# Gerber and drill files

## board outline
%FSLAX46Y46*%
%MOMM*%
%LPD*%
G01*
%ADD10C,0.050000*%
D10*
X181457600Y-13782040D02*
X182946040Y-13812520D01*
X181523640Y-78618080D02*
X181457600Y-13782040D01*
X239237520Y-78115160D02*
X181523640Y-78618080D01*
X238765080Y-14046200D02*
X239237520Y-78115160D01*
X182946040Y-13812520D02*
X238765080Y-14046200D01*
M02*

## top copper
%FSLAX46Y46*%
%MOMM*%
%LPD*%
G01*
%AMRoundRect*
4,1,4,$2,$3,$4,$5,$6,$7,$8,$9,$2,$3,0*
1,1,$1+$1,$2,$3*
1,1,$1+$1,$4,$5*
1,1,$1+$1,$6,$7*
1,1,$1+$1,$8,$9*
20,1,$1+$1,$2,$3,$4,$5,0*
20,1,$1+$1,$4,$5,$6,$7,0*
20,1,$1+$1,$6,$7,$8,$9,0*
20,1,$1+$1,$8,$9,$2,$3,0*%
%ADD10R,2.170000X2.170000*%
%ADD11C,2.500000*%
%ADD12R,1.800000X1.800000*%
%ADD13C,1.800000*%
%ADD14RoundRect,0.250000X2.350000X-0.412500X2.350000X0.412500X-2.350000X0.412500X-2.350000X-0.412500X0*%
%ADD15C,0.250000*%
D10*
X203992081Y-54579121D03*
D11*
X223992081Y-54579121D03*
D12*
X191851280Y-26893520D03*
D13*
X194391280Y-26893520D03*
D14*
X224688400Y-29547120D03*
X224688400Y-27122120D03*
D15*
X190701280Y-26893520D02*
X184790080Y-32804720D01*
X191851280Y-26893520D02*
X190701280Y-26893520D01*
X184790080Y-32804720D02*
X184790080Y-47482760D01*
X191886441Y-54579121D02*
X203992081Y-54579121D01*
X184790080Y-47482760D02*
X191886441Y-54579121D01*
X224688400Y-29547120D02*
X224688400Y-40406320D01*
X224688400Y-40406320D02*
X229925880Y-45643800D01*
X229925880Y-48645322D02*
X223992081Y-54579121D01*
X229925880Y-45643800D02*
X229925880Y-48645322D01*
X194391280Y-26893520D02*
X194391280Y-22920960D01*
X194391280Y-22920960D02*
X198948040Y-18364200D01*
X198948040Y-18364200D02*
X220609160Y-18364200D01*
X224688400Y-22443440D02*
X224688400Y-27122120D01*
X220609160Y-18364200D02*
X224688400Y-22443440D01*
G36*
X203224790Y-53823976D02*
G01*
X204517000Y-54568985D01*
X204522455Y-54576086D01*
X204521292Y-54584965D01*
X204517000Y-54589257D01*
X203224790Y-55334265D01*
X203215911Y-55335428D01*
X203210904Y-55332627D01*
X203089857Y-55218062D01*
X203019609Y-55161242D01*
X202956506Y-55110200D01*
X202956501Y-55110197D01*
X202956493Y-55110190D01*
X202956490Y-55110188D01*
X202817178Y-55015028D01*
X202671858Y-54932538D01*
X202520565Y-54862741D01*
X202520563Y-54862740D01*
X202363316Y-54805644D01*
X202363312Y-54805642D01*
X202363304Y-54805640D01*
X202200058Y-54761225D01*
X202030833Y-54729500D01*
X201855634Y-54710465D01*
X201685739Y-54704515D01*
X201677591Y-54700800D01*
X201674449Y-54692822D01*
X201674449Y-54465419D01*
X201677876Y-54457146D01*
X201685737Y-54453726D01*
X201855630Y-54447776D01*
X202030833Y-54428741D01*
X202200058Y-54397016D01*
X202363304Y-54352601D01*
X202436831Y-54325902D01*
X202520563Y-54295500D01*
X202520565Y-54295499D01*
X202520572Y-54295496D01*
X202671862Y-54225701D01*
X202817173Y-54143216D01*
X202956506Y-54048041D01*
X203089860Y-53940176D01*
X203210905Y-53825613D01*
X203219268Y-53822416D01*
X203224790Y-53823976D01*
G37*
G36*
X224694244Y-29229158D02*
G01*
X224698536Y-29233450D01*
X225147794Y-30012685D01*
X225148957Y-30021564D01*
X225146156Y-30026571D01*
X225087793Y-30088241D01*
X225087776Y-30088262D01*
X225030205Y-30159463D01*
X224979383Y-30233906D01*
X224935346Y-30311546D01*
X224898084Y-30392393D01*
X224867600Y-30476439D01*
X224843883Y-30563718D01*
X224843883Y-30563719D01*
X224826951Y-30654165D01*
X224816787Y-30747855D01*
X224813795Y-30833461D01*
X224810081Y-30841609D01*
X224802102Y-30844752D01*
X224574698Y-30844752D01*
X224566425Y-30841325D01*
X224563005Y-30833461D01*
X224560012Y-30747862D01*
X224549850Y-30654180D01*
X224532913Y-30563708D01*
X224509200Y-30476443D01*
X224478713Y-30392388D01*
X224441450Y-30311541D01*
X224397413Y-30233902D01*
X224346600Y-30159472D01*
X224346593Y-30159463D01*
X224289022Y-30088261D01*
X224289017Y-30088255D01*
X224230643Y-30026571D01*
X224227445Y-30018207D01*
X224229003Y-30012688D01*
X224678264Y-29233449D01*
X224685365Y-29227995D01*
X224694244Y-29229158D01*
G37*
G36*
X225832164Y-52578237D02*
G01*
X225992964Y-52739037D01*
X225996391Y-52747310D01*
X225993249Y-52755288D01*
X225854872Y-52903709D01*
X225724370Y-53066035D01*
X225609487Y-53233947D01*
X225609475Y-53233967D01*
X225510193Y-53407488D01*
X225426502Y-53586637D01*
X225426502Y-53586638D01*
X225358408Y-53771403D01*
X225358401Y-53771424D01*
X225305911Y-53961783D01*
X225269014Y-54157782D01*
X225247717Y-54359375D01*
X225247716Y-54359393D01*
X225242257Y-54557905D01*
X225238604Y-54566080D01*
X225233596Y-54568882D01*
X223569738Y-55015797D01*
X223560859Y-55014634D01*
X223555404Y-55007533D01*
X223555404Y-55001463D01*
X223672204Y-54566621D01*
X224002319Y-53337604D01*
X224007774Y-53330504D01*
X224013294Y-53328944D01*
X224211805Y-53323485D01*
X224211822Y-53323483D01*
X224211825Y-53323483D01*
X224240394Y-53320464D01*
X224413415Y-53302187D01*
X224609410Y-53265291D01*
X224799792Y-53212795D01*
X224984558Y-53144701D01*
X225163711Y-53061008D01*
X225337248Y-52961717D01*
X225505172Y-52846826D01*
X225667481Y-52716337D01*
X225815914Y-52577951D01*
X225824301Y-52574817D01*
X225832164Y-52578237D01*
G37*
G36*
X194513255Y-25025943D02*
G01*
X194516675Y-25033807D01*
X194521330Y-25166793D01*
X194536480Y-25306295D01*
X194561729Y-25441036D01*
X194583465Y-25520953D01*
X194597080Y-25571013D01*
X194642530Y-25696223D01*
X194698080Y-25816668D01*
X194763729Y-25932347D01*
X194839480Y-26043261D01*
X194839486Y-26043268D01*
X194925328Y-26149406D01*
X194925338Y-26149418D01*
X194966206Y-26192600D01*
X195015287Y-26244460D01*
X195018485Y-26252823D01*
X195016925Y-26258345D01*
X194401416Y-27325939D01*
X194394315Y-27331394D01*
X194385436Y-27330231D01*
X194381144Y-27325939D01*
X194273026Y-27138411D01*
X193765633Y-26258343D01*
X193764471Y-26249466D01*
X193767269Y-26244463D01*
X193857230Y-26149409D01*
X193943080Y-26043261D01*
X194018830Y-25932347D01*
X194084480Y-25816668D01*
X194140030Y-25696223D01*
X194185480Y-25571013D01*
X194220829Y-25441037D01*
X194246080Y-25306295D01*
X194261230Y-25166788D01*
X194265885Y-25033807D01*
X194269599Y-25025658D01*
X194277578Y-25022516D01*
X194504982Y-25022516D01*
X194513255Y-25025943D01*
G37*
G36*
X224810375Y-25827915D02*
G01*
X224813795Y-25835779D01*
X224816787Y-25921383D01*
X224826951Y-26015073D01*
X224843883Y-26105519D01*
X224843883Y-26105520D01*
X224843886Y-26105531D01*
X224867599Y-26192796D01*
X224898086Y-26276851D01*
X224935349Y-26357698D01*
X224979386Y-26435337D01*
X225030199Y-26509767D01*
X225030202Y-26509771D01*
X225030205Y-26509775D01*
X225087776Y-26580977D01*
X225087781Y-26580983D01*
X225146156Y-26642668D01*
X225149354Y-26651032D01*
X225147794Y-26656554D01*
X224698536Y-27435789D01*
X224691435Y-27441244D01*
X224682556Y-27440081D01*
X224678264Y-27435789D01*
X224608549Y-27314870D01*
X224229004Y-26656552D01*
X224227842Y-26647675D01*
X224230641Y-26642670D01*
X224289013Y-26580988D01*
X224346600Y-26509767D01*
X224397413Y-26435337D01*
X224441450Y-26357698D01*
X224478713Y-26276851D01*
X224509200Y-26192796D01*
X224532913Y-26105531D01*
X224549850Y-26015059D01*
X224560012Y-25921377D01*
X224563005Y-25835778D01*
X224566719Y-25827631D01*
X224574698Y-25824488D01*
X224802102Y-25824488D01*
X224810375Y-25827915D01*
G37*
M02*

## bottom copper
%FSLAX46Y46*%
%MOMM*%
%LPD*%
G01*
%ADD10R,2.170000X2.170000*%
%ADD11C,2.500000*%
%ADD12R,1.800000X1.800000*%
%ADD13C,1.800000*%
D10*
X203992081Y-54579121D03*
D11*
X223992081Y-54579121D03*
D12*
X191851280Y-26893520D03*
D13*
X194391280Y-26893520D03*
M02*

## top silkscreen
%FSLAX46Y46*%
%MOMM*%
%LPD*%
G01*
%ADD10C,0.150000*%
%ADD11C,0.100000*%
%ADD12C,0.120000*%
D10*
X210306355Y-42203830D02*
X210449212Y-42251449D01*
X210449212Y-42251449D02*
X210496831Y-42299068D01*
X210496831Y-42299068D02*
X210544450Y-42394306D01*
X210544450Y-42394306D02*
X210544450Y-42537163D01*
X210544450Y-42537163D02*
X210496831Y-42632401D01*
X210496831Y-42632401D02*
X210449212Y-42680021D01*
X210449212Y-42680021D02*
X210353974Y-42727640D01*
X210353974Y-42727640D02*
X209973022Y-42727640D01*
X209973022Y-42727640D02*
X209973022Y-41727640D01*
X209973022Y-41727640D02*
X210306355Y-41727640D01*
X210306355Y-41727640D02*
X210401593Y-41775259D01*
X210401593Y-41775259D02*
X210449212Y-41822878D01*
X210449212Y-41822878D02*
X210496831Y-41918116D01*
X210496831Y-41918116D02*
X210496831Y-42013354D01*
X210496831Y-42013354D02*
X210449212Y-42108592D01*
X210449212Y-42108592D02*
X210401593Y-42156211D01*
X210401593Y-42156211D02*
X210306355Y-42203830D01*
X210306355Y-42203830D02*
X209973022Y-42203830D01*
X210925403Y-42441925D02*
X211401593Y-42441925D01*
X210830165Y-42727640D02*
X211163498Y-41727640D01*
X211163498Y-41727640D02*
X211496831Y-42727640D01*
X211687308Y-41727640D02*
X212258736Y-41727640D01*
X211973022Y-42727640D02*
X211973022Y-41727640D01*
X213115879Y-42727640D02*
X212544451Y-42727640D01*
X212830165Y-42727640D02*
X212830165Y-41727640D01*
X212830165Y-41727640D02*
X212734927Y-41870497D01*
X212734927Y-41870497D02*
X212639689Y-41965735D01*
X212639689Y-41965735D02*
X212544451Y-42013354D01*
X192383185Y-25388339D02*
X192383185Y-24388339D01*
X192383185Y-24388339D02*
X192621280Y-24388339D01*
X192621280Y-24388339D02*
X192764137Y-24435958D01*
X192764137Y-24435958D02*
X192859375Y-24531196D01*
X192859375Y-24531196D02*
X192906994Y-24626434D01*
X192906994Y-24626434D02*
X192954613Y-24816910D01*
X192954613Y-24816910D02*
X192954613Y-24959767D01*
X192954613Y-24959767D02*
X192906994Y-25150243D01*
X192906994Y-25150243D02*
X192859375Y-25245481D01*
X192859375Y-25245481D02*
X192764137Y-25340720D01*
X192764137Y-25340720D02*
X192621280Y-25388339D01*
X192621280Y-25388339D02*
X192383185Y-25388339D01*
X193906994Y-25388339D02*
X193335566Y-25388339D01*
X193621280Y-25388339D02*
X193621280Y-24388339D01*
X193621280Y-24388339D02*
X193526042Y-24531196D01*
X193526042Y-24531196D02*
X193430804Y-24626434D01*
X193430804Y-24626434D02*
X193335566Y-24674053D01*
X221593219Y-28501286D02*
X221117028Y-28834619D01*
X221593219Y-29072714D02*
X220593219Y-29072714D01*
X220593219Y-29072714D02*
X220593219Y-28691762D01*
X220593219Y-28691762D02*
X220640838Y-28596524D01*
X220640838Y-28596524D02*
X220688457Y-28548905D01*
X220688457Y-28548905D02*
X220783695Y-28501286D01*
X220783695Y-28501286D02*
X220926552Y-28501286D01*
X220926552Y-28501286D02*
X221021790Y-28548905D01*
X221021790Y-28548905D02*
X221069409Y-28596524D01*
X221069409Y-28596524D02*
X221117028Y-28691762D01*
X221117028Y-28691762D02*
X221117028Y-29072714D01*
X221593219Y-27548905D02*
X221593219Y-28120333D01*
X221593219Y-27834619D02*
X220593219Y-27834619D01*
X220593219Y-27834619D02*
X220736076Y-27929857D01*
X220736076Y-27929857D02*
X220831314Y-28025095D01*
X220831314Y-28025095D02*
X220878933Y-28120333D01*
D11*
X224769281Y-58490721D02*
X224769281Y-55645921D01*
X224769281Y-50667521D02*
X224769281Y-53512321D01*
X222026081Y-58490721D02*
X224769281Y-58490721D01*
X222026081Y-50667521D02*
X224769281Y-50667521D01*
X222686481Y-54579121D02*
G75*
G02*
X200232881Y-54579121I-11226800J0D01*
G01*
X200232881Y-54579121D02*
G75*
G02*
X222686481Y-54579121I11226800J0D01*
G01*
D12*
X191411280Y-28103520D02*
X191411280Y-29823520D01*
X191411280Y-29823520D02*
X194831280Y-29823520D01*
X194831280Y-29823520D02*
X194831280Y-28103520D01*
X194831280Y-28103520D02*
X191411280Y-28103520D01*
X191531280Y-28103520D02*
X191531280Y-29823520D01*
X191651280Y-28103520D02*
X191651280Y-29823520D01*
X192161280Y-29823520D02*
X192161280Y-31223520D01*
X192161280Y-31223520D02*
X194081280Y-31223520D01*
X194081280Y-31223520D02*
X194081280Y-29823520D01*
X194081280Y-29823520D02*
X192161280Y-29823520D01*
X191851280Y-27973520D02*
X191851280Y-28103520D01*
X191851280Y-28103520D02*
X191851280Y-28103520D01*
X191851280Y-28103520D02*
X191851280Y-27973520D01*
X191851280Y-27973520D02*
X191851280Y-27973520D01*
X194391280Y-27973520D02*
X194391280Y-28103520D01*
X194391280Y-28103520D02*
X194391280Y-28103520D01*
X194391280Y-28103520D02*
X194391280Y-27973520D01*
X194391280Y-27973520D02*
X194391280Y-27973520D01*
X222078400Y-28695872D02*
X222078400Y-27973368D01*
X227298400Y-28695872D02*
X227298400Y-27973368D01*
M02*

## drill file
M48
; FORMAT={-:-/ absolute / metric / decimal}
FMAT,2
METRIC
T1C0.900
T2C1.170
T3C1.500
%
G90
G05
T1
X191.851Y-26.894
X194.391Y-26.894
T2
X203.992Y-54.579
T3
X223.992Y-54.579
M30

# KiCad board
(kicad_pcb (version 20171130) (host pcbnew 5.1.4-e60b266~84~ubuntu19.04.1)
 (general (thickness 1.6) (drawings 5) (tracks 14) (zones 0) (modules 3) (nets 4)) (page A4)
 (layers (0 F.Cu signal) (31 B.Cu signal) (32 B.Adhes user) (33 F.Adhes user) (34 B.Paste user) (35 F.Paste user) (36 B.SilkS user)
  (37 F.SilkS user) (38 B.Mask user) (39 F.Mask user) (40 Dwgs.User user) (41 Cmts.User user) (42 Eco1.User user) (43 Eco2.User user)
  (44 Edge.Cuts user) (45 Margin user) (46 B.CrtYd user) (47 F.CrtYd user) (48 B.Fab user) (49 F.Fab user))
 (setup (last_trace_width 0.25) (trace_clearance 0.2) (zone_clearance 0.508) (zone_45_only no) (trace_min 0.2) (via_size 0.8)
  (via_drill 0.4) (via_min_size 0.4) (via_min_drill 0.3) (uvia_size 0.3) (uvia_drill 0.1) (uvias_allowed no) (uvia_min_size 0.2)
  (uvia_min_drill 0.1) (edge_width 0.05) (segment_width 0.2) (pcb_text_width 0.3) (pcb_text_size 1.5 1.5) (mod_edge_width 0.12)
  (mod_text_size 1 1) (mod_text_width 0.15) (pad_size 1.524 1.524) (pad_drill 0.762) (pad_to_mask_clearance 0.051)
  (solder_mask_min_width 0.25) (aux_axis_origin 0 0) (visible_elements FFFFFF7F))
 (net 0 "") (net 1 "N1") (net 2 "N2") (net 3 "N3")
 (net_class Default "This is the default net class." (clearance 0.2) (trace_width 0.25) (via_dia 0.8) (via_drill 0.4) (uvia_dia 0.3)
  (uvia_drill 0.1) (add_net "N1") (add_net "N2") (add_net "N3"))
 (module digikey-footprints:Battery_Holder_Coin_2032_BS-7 (layer F.Cu) (at 203.992081 54.579121)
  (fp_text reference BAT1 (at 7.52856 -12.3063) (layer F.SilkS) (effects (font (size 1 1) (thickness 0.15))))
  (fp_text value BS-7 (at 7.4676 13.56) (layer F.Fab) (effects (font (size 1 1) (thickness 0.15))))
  (fp_line (start 20.7772 3.9116) (end 20.7772 1.0668) (layer F.SilkS) (width 0.1))
  (fp_line (start 20.7772 -3.9116) (end 20.7772 -1.0668) (layer F.SilkS) (width 0.1))
  (fp_line (start 18.034 3.9116) (end 20.7772 3.9116) (layer F.SilkS) (width 0.1))
  (fp_line (start 18.034 -3.9116) (end 20.7772 -3.9116) (layer F.SilkS) (width 0.1))
  (fp_circle (center 7.4676 0) (end -3.7592 0) (layer F.SilkS) (width 0.1))
  (pad Neg thru_hole rect (at 0 0) (size 2.17 2.17) (drill 1.17) (layers *.Cu *.Mask) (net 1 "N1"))
  (pad Pos thru_hole circle (at 20 0) (size 2.5 2.5) (drill 1.5) (layers *.Cu *.Mask) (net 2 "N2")))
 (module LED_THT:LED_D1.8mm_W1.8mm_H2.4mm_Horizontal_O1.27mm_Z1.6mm (layer F.Cu) (at 191.85128 26.89352)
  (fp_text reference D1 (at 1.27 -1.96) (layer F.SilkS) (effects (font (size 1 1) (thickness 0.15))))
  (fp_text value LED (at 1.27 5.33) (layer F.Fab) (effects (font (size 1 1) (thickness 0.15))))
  (fp_line (start -0.44 1.21) (end -0.44 2.93) (layer F.SilkS) (width 0.12))
  (fp_line (start -0.44 2.93) (end 2.98 2.93) (layer F.SilkS) (width 0.12))
  (fp_line (start 2.98 2.93) (end 2.98 1.21) (layer F.SilkS) (width 0.12))
  (fp_line (start 2.98 1.21) (end -0.44 1.21) (layer F.SilkS) (width 0.12))
  (fp_line (start -0.32 1.21) (end -0.32 2.93) (layer F.SilkS) (width 0.12))
  (fp_line (start -0.2 1.21) (end -0.2 2.93) (layer F.SilkS) (width 0.12))
  (fp_line (start 0.31 2.93) (end 0.31 4.33) (layer F.SilkS) (width 0.12))
  (fp_line (start 0.31 4.33) (end 2.23 4.33) (layer F.SilkS) (width 0.12))
  (fp_line (start 2.23 4.33) (end 2.23 2.93) (layer F.SilkS) (width 0.12))
  (fp_line (start 2.23 2.93) (end 0.31 2.93) (layer F.SilkS) (width 0.12))
  (fp_line (start 0 1.08) (end 0 1.21) (layer F.SilkS) (width 0.12))
  (fp_line (start 0 1.21) (end 0 1.21) (layer F.SilkS) (width 0.12))
  (fp_line (start 0 1.21) (end 0 1.08) (layer F.SilkS) (width 0.12))
  (fp_line (start 0 1.08) (end 0 1.08) (layer F.SilkS) (width 0.12))
  (fp_line (start 2.54 1.08) (end 2.54 1.21) (layer F.SilkS) (width 0.12))
  (fp_line (start 2.54 1.21) (end 2.54 1.21) (layer F.SilkS) (width 0.12))
  (fp_line (start 2.54 1.21) (end 2.54 1.08) (layer F.SilkS) (width 0.12))
  (fp_line (start 2.54 1.08) (end 2.54 1.08) (layer F.SilkS) (width 0.12))
  (pad 1 thru_hole rect (at 0 0) (size 1.8 1.8) (drill 0.9) (layers *.Cu *.Mask) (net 1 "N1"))
  (pad 2 thru_hole circle (at 2.54 0) (size 1.8 1.8) (drill 0.9) (layers *.Cu *.Mask) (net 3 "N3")))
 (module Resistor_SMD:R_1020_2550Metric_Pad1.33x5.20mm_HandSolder (layer F.Cu) (at 224.6884 28.33462 90)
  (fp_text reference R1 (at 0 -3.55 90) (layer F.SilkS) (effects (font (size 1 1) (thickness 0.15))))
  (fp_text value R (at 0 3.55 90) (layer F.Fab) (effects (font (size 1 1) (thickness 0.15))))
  (fp_line (start -0.361252 -2.61) (end 0.361252 -2.61) (layer F.SilkS) (width 0.12))
  (fp_line (start -0.361252 2.61) (end 0.361252 2.61) (layer F.SilkS) (width 0.12))
  (pad 1 smd roundrect (at -1.2125 0 90) (size 1.325 5.2) (layers F.Cu F.Paste F.Mask) (roundrect_rratio 0.188679) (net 2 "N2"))
  (pad 2 smd roundrect (at 1.2125 0 90) (size 1.325 5.2) (layers F.Cu F.Paste F.Mask) (roundrect_rratio 0.188679) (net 3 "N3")))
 (gr_line (start 181.4576 13.78204) (end 182.94604 13.81252) (layer Edge.Cuts) (width 0.05))
 (gr_line (start 181.52364 78.61808) (end 181.4576 13.78204) (layer Edge.Cuts) (width 0.05))
 (gr_line (start 239.23752 78.11516) (end 181.52364 78.61808) (layer Edge.Cuts) (width 0.05))
 (gr_line (start 238.76508 14.0462) (end 239.23752 78.11516) (layer Edge.Cuts) (width 0.05))
 (gr_line (start 182.94604 13.81252) (end 238.76508 14.0462) (layer Edge.Cuts) (width 0.05))
 (segment (start 190.70128 26.89352) (end 184.79008 32.80472) (width 0.25) (layer F.Cu) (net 1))
 (segment (start 191.85128 26.89352) (end 190.70128 26.89352) (width 0.25) (layer F.Cu) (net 1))
 (segment (start 184.79008 32.80472) (end 184.79008 47.48276) (width 0.25) (layer F.Cu) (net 1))
 (segment (start 191.886441 54.579121) (end 203.992081 54.579121) (width 0.25) (layer F.Cu) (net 1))
 (segment (start 184.79008 47.48276) (end 191.886441 54.579121) (width 0.25) (layer F.Cu) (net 1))
 (segment (start 224.6884 29.54712) (end 224.6884 40.40632) (width 0.25) (layer F.Cu) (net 2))
 (segment (start 224.6884 40.40632) (end 229.92588 45.6438) (width 0.25) (layer F.Cu) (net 2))
 (segment (start 229.92588 48.645322) (end 223.992081 54.579121) (width 0.25) (layer F.Cu) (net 2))
 (segment (start 229.92588 45.6438) (end 229.92588 48.645322) (width 0.25) (layer F.Cu) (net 2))
 (segment (start 194.39128 26.89352) (end 194.39128 22.92096) (width 0.25) (layer F.Cu) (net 3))
 (segment (start 194.39128 22.92096) (end 198.94804 18.3642) (width 0.25) (layer F.Cu) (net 3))
 (segment (start 198.94804 18.3642) (end 220.60916 18.3642) (width 0.25) (layer F.Cu) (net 3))
 (segment (start 224.6884 22.44344) (end 224.6884 27.12212) (width 0.25) (layer F.Cu) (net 3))
 (segment (start 220.60916 18.3642) (end 224.6884 22.44344) (width 0.25) (layer F.Cu) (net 3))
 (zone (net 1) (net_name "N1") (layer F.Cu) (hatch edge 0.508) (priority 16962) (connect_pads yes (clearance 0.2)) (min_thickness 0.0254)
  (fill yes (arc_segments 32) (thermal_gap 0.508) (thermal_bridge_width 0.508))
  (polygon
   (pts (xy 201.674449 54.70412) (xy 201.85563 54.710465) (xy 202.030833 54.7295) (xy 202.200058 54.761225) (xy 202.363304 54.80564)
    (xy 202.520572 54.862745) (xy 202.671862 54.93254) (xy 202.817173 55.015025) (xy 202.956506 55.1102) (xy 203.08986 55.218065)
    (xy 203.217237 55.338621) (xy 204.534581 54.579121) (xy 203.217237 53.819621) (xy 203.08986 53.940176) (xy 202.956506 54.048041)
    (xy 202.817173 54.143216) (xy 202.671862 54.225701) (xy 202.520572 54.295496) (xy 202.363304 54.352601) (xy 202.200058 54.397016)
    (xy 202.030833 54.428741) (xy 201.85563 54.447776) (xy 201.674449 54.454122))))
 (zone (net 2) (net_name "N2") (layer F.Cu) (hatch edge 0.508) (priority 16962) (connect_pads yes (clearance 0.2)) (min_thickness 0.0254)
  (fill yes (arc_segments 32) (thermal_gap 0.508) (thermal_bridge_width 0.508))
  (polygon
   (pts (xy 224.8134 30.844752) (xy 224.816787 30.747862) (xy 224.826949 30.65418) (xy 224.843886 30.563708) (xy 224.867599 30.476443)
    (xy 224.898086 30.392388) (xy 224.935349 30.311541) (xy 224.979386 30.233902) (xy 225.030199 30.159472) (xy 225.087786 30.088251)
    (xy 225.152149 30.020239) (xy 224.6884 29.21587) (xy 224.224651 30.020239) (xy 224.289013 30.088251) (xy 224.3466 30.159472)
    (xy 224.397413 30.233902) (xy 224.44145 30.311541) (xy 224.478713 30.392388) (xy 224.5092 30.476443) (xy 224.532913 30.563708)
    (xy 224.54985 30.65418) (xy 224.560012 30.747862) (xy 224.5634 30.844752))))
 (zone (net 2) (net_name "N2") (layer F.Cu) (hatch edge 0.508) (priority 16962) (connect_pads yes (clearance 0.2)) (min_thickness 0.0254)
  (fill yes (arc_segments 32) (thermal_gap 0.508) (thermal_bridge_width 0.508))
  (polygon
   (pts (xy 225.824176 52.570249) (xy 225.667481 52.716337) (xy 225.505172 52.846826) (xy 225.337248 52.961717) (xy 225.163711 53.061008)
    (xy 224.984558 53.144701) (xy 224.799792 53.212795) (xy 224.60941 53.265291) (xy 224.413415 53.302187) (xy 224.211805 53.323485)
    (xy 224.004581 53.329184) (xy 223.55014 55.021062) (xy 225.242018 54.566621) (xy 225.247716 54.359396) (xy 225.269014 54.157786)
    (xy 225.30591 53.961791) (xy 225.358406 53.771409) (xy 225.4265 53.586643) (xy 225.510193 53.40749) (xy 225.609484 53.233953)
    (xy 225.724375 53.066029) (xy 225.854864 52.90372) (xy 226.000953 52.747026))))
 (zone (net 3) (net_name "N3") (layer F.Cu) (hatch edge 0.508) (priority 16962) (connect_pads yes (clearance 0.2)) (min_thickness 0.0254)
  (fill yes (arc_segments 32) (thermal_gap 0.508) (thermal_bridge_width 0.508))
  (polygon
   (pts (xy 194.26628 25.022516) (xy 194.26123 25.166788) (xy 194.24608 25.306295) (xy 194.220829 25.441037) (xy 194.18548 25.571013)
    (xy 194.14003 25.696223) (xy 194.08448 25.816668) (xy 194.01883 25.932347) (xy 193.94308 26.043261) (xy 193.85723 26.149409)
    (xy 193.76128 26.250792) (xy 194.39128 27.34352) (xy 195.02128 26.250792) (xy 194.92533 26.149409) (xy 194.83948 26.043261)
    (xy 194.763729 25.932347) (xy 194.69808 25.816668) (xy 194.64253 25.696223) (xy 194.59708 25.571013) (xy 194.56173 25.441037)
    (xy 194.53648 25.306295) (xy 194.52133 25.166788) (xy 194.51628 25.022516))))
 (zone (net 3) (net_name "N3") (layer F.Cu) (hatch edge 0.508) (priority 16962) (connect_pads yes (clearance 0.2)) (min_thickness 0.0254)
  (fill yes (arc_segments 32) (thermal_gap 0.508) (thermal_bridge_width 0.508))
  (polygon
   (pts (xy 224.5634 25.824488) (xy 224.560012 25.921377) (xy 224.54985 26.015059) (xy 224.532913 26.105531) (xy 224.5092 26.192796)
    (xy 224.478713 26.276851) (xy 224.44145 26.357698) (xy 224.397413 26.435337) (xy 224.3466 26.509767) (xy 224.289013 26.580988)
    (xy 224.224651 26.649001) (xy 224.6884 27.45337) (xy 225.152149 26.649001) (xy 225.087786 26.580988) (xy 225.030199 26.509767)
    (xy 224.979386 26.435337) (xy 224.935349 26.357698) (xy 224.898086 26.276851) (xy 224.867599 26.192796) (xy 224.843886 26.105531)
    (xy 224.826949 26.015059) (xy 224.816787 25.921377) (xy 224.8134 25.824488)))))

